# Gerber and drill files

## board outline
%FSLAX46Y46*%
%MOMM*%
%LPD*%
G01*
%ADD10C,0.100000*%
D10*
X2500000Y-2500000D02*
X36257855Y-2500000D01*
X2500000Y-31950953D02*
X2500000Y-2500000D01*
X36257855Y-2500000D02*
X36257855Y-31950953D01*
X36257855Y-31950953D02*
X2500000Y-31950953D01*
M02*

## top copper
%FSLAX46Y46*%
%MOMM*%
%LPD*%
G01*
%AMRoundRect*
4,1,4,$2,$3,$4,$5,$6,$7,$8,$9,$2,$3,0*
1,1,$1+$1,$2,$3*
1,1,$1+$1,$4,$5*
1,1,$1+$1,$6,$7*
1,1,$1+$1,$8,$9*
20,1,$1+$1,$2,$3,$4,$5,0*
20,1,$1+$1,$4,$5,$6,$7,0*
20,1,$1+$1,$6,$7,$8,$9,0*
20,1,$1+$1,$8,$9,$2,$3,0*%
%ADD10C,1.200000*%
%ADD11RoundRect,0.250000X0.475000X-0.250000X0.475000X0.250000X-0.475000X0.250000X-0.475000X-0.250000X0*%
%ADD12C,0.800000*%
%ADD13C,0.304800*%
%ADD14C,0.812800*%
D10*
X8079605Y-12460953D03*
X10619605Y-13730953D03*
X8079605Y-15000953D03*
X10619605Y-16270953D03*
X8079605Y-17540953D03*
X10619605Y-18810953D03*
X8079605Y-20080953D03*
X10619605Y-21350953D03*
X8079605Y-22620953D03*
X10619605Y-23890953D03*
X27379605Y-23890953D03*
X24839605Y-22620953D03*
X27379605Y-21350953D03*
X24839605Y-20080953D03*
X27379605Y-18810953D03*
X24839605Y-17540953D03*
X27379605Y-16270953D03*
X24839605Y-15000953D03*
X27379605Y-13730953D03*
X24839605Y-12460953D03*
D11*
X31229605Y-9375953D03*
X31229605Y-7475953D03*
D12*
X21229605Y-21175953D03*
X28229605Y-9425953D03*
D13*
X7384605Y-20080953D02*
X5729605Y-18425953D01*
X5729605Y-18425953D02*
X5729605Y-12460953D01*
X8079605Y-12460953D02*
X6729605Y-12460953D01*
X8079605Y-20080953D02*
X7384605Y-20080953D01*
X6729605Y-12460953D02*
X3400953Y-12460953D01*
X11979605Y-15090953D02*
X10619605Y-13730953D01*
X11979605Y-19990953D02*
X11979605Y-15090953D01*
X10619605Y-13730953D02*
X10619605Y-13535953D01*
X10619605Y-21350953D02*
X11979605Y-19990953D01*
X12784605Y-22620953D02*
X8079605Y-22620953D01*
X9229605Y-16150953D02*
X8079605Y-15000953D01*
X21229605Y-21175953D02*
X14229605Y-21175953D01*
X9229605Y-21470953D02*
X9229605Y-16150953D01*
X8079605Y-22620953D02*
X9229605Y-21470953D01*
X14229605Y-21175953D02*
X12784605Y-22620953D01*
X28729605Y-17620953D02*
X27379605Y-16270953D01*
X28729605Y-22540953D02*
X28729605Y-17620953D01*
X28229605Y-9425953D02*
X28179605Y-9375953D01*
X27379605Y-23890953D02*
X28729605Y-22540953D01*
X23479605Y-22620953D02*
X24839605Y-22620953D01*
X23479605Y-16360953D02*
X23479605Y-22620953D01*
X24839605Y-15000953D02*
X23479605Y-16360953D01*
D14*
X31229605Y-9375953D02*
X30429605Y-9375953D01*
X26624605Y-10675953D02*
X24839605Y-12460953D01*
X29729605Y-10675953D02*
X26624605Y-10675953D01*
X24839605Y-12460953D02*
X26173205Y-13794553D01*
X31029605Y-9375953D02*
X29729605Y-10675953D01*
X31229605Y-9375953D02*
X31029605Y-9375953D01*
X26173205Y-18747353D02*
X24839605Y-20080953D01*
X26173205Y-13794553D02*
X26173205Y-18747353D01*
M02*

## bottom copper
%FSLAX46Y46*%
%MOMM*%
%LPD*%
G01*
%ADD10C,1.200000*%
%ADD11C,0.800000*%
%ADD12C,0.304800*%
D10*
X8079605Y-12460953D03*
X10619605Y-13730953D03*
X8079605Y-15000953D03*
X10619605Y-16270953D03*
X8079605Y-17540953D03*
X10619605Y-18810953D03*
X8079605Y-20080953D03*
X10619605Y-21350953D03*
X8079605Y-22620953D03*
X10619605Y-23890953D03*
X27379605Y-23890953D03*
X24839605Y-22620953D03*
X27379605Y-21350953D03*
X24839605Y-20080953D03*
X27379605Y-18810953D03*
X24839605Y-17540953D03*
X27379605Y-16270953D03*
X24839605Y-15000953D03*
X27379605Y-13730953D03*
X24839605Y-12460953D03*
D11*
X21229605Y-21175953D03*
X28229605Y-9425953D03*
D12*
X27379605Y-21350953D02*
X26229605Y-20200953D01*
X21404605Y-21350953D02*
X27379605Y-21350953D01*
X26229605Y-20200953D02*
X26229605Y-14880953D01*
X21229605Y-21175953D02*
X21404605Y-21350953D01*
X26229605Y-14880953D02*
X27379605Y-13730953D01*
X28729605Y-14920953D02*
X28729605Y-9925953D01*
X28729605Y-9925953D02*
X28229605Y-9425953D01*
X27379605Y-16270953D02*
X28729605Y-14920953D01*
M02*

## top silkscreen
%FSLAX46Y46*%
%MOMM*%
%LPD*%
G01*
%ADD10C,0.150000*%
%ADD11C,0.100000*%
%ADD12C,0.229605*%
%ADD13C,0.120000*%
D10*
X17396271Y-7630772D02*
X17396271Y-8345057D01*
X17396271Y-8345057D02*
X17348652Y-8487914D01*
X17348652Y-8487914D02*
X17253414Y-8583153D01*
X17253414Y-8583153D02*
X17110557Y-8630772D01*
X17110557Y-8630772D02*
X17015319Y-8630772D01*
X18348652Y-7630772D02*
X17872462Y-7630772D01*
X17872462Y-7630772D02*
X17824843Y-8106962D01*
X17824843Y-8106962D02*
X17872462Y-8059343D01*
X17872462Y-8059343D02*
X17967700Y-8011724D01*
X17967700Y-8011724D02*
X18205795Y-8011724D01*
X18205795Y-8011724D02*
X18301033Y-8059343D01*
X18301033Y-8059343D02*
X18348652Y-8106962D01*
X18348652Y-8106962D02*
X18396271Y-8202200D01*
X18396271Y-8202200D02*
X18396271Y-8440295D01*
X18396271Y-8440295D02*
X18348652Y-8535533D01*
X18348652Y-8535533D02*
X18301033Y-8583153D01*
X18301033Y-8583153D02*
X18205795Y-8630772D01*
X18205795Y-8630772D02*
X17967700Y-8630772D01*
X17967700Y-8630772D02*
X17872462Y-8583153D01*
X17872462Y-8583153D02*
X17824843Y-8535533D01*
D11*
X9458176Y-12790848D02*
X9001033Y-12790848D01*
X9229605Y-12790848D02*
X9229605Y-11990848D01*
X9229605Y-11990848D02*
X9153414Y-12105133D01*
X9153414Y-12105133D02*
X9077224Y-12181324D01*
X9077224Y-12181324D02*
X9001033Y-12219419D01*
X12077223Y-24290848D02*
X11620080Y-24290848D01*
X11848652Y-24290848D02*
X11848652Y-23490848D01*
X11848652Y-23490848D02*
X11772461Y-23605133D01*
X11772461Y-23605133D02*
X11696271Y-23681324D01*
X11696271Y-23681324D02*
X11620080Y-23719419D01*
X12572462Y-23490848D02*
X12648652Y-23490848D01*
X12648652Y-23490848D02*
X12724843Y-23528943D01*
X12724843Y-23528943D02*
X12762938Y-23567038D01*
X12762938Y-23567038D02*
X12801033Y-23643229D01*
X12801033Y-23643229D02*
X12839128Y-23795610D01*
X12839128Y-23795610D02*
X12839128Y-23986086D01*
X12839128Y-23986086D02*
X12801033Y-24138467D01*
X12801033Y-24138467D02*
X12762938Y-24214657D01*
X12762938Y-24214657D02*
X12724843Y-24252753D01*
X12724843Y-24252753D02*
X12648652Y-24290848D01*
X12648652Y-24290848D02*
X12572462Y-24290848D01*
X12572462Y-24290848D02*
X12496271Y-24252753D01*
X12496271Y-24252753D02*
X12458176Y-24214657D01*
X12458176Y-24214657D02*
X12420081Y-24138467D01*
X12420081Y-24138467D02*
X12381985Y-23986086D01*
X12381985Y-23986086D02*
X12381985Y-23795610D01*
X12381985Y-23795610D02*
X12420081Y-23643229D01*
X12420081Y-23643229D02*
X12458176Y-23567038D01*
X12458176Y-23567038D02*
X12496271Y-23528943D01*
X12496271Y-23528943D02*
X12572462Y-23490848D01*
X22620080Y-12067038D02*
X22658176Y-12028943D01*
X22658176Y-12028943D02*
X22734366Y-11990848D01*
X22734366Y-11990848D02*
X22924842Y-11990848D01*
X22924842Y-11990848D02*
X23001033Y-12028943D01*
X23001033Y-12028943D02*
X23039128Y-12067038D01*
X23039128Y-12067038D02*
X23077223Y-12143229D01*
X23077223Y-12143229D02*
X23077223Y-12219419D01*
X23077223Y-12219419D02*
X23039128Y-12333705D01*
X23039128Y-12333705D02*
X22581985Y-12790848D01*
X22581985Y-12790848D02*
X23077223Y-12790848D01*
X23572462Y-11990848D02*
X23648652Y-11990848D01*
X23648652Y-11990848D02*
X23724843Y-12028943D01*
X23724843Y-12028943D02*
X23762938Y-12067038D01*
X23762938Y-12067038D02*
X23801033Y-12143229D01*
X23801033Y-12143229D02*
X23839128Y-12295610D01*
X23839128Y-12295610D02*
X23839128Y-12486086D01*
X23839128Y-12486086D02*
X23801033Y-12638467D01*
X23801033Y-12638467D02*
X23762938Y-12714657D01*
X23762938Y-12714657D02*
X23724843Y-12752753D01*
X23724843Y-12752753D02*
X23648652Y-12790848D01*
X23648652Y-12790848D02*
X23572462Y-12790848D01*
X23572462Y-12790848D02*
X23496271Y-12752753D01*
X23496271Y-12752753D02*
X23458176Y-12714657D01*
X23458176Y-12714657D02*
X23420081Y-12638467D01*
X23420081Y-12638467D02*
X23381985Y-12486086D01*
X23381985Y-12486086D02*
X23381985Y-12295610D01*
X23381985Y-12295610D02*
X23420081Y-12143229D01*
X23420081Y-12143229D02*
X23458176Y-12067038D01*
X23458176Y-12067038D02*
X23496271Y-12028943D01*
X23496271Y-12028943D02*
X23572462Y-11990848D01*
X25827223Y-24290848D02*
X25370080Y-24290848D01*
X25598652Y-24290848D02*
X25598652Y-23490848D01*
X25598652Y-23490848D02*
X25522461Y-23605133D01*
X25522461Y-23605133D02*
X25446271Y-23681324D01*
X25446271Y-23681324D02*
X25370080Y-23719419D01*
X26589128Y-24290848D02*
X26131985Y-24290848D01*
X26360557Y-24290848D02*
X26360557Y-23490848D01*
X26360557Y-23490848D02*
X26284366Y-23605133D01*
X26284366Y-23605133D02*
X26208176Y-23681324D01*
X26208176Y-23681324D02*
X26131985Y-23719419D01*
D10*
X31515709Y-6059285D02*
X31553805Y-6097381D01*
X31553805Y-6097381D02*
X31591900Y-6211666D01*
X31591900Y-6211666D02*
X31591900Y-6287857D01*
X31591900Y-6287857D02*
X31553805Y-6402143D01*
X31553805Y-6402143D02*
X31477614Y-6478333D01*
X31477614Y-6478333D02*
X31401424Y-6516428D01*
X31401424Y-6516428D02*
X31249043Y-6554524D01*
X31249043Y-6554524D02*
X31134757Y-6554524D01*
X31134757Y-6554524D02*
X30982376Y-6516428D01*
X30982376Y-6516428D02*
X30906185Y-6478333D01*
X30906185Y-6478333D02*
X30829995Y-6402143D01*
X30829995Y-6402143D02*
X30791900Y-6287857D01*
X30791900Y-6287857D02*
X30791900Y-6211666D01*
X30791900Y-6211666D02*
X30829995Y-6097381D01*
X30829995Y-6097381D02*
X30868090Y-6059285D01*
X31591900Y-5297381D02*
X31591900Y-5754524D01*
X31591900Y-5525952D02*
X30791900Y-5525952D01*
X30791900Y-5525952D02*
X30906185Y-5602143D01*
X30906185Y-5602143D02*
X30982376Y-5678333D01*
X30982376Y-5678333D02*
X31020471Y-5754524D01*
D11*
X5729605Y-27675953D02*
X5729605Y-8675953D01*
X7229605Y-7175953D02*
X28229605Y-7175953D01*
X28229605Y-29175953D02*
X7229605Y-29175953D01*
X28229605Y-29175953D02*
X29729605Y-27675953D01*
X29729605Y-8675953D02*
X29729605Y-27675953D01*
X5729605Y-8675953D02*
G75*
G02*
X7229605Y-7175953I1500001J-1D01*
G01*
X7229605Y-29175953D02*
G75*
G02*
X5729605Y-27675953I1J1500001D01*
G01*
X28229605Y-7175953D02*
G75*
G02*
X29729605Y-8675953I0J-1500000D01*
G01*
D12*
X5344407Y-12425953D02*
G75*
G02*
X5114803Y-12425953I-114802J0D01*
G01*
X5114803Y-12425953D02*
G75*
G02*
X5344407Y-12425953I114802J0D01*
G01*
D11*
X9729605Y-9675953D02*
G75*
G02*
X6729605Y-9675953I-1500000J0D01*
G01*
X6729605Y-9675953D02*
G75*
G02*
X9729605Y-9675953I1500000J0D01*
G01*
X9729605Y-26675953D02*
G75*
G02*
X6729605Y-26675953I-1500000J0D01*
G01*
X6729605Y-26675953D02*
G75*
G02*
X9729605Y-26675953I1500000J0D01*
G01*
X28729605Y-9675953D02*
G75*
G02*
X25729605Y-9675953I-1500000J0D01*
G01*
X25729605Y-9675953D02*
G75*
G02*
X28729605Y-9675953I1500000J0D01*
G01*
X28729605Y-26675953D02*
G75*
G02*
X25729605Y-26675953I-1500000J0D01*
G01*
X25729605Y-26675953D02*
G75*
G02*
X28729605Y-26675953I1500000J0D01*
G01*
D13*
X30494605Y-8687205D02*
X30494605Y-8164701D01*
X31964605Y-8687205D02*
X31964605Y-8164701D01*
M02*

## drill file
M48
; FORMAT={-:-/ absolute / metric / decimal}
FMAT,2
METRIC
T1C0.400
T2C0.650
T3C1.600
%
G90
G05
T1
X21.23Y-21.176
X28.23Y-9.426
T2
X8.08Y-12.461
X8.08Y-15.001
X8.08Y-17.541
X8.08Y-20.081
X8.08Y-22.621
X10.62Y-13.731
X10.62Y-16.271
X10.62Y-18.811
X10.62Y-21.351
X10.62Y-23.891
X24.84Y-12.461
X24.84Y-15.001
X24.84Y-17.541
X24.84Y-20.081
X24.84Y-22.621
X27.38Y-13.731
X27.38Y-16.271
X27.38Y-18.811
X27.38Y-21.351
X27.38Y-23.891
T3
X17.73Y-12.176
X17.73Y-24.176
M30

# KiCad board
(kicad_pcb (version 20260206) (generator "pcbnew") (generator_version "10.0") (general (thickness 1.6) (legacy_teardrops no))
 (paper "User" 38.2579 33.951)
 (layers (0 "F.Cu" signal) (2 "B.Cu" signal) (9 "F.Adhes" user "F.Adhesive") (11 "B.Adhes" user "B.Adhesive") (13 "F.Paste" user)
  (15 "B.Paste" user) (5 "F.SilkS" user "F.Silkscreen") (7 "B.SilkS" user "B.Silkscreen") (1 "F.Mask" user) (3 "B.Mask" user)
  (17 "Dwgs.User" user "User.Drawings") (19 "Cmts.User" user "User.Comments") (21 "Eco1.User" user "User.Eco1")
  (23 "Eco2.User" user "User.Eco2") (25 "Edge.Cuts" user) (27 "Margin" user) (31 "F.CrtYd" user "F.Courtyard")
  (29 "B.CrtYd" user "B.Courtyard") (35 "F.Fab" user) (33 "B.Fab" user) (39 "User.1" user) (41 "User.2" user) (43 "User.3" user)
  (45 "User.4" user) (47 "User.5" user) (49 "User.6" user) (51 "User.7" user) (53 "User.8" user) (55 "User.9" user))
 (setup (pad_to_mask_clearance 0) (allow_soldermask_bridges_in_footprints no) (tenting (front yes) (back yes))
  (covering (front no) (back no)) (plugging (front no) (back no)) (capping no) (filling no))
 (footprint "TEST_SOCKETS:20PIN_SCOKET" (layer "F.Cu") (at 17.729605 18.175953)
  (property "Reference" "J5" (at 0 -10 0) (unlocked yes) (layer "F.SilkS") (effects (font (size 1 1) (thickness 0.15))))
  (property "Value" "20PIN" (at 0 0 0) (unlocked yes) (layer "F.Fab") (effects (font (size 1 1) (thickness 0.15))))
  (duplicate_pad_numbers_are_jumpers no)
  (fp_line (start -12 9.5) (end -12 -9.5) (stroke (width 0.1) (type default)) (layer "F.SilkS"))
  (fp_line (start -10.5 -11) (end 10.5 -11) (stroke (width 0.1) (type default)) (layer "F.SilkS"))
  (fp_line (start 10.5 11) (end -10.5 11) (stroke (width 0.1) (type default)) (layer "F.SilkS"))
  (fp_line (start 10.5 11) (end 12 9.5) (stroke (width 0.1) (type default)) (layer "F.SilkS"))
  (fp_line (start 12 -9.5) (end 12 9.5) (stroke (width 0.1) (type default)) (layer "F.SilkS"))
  (fp_arc (start -12 -9.5) (mid -11.56066 -10.56066) (end -10.5 -11) (stroke (width 0.1) (type default)) (layer "F.SilkS"))
  (fp_arc (start -10.5 11) (mid -11.56066 10.56066) (end -12 9.5) (stroke (width 0.1) (type default)) (layer "F.SilkS"))
  (fp_arc (start 10.5 -11) (mid 11.56066 -10.56066) (end 12 -9.5) (stroke (width 0.1) (type default)) (layer "F.SilkS"))
  (fp_circle (center -12.5 -5.75) (end -12.320395 -5.75) (stroke (width 0.1) (type solid)) (fill yes) (layer "F.SilkS"))
  (fp_circle (center -9.5 -8.5) (end -8 -8.5) (stroke (width 0.1) (type default)) (fill no) (layer "F.SilkS"))
  (fp_circle (center -9.5 8.5) (end -8 8.5) (stroke (width 0.1) (type default)) (fill no) (layer "F.SilkS"))
  (fp_circle (center 9.5 -8.5) (end 8 -8.5) (stroke (width 0.1) (type default)) (fill no) (layer "F.SilkS"))
  (fp_circle (center 9.5 8.5) (end 8 8.5) (stroke (width 0.1) (type default)) (fill no) (layer "F.SilkS"))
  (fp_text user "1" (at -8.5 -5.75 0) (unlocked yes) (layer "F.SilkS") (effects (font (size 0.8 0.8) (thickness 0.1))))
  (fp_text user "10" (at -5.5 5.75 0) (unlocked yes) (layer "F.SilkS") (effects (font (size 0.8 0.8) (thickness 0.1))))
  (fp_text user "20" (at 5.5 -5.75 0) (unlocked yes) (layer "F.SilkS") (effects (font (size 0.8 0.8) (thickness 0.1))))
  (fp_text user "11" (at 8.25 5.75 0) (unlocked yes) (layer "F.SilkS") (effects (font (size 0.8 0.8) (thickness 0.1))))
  (pad "" np_thru_hole circle (at 0 -6) (size 1.6 1.6) (drill 1.6) (layers "*.Cu" "*.Mask"))
  (pad "" np_thru_hole circle (at 0 6) (size 1.6 1.6) (drill 1.6) (layers "*.Cu" "*.Mask"))
  (pad "1" thru_hole circle (at -9.65 -5.715) (size 1.2 1.2) (drill 0.65) (layers "*.Cu" "*.Mask") (remove_unused_layers no) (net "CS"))
  (pad "2" thru_hole circle (at -7.11 -4.445) (size 1.2 1.2) (drill 0.65) (layers "*.Cu" "*.Mask") (remove_unused_layers no) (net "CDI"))
  (pad "3" thru_hole circle (at -9.65 -3.175) (size 1.2 1.2) (drill 0.65) (layers "*.Cu" "*.Mask") (remove_unused_layers no) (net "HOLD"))
  (pad "4" thru_hole circle (at -7.11 -1.905) (size 1.2 1.2) (drill 0.65) (layers "*.Cu" "*.Mask") (remove_unused_layers no)
   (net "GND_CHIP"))
  (pad "5" thru_hole circle (at -9.65 -0.635) (size 1.2 1.2) (drill 0.65) (layers "*.Cu" "*.Mask") (remove_unused_layers no)
   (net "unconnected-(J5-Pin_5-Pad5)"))
  (pad "6" thru_hole circle (at -7.11 0.635) (size 1.2 1.2) (drill 0.65) (layers "*.Cu" "*.Mask") (remove_unused_layers no)
   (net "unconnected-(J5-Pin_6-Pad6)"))
  (pad "7" thru_hole circle (at -9.65 1.905) (size 1.2 1.2) (drill 0.65) (layers "*.Cu" "*.Mask") (remove_unused_layers no) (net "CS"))
  (pad "8" thru_hole circle (at -7.11 3.175) (size 1.2 1.2) (drill 0.65) (layers "*.Cu" "*.Mask") (remove_unused_layers no) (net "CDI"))
  (pad "9" thru_hole circle (at -9.65 4.445) (size 1.2 1.2) (drill 0.65) (layers "*.Cu" "*.Mask") (remove_unused_layers no) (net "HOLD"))
  (pad "10" thru_hole circle (at -7.11 5.715) (size 1.2 1.2) (drill 0.65) (layers "*.Cu" "*.Mask") (remove_unused_layers no)
   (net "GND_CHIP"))
  (pad "11" thru_hole circle (at 9.65 5.715 180) (size 1.2 1.2) (drill 0.65) (layers "*.Cu" "*.Mask") (remove_unused_layers no) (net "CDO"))
  (pad "12" thru_hole circle (at 7.11 4.445 180) (size 1.2 1.2) (drill 0.65) (layers "*.Cu" "*.Mask") (remove_unused_layers no) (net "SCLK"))
  (pad "13" thru_hole circle (at 9.65 3.175 180) (size 1.2 1.2) (drill 0.65) (layers "*.Cu" "*.Mask") (remove_unused_layers no) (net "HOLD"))
  (pad "14" thru_hole circle (at 7.11 1.905 180) (size 1.2 1.2) (drill 0.65) (layers "*.Cu" "*.Mask") (remove_unused_layers no)
   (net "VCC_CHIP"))
  (pad "15" thru_hole circle (at 9.65 0.635 180) (size 1.2 1.2) (drill 0.65) (layers "*.Cu" "*.Mask") (remove_unused_layers no)
   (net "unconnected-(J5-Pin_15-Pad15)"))
  (pad "16" thru_hole circle (at 7.11 -0.635 180) (size 1.2 1.2) (drill 0.65) (layers "*.Cu" "*.Mask") (remove_unused_layers no)
   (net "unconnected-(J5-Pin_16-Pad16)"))
  (pad "17" thru_hole circle (at 9.65 -1.905 180) (size 1.2 1.2) (drill 0.65) (layers "*.Cu" "*.Mask") (remove_unused_layers no) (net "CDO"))
  (pad "18" thru_hole circle (at 7.11 -3.175 180) (size 1.2 1.2) (drill 0.65) (layers "*.Cu" "*.Mask") (remove_unused_layers no)
   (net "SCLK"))
  (pad "19" thru_hole circle (at 9.65 -4.445 180) (size 1.2 1.2) (drill 0.65) (layers "*.Cu" "*.Mask") (remove_unused_layers no)
   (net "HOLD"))
  (pad "20" thru_hole circle (at 7.11 -5.715 180) (size 1.2 1.2) (drill 0.65) (layers "*.Cu" "*.Mask") (remove_unused_layers no)
   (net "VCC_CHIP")))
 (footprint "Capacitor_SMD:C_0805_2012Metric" (layer "F.Cu") (at 31.229605 8.425953 90)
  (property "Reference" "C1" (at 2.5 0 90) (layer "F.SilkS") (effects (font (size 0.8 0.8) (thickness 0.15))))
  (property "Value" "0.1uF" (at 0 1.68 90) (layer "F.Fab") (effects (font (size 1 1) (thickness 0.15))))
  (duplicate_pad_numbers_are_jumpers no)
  (fp_line (start -0.261252 -0.735) (end 0.261252 -0.735) (stroke (width 0.12) (type solid)) (layer "F.SilkS"))
  (fp_line (start -0.261252 0.735) (end 0.261252 0.735) (stroke (width 0.12) (type solid)) (layer "F.SilkS"))
  (pad "1" smd roundrect (at -0.95 0 90) (size 1 1.45) (layers "F.Cu" "F.Mask" "F.Paste") (roundrect_rratio 0.25) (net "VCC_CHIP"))
  (pad "2" smd roundrect (at 0.95 0 90) (size 1 1.45) (layers "F.Cu" "F.Mask" "F.Paste") (roundrect_rratio 0.25) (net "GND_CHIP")))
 (gr_line (start 2.5 2.5) (end 36.257855 2.5) (stroke (width 0.1) (type default)) (layer "Edge.Cuts"))
 (gr_line (start 2.5 31.950953) (end 2.5 2.5) (stroke (width 0.1) (type default)) (layer "Edge.Cuts"))
 (gr_line (start 36.257855 2.5) (end 36.257855 31.950953) (stroke (width 0.1) (type default)) (layer "Edge.Cuts"))
 (gr_line (start 36.257855 31.950953) (end 2.5 31.950953) (stroke (width 0.1) (type default)) (layer "Edge.Cuts"))
 (segment (start 7.384605 20.080953) (end 5.729605 18.425953) (width 0.3048) (layer "F.Cu") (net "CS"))
 (segment (start 5.729605 18.425953) (end 5.729605 12.460953) (width 0.3048) (layer "F.Cu") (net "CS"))
 (segment (start 8.079605 12.460953) (end 6.729605 12.460953) (width 0.3048) (layer "F.Cu") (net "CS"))
 (segment (start 8.079605 20.080953) (end 7.384605 20.080953) (width 0.3048) (layer "F.Cu") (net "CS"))
 (segment (start 6.729605 12.460953) (end 3.400953 12.460953) (width 0.3048) (layer "F.Cu") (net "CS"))
 (segment (start 11.979605 15.090953) (end 10.619605 13.730953) (width 0.3048) (layer "F.Cu") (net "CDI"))
 (segment (start 11.979605 19.990953) (end 11.979605 15.090953) (width 0.3048) (layer "F.Cu") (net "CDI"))
 (segment (start 10.619605 13.730953) (end 10.619605 13.535953) (width 0.3048) (layer "F.Cu") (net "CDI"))
 (segment (start 10.619605 21.350953) (end 11.979605 19.990953) (width 0.3048) (layer "F.Cu") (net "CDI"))
 (segment (start 12.784605 22.620953) (end 8.079605 22.620953) (width 0.3048) (layer "F.Cu") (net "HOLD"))
 (segment (start 9.229605 16.150953) (end 8.079605 15.000953) (width 0.3048) (layer "F.Cu") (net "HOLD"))
 (segment (start 21.229605 21.175953) (end 14.229605 21.175953) (width 0.3048) (layer "F.Cu") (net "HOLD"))
 (segment (start 9.229605 21.470953) (end 9.229605 16.150953) (width 0.3048) (layer "F.Cu") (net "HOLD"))
 (segment (start 8.079605 22.620953) (end 9.229605 21.470953) (width 0.3048) (layer "F.Cu") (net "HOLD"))
 (segment (start 14.229605 21.175953) (end 12.784605 22.620953) (width 0.3048) (layer "F.Cu") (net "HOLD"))
 (via (at 21.229605 21.175953) (size 0.8) (drill 0.4) (layers "F.Cu" "B.Cu") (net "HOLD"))
 (segment (start 27.379605 21.350953) (end 26.229605 20.200953) (width 0.3048) (layer "B.Cu") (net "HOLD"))
 (segment (start 21.404605 21.350953) (end 27.379605 21.350953) (width 0.3048) (layer "B.Cu") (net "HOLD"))
 (segment (start 26.229605 20.200953) (end 26.229605 14.880953) (width 0.3048) (layer "B.Cu") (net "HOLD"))
 (segment (start 21.229605 21.175953) (end 21.404605 21.350953) (width 0.3048) (layer "B.Cu") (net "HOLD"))
 (segment (start 26.229605 14.880953) (end 27.379605 13.730953) (width 0.3048) (layer "B.Cu") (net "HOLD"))
 (segment (start 28.729605 17.620953) (end 27.379605 16.270953) (width 0.3048) (layer "F.Cu") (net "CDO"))
 (segment (start 28.729605 22.540953) (end 28.729605 17.620953) (width 0.3048) (layer "F.Cu") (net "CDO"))
 (segment (start 28.229605 9.425953) (end 28.179605 9.375953) (width 0.3048) (layer "F.Cu") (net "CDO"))
 (segment (start 27.379605 23.890953) (end 28.729605 22.540953) (width 0.3048) (layer "F.Cu") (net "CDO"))
 (via (at 28.229605 9.425953) (size 0.8) (drill 0.4) (layers "F.Cu" "B.Cu") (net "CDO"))
 (segment (start 28.729605 14.920953) (end 28.729605 9.925953) (width 0.3048) (layer "B.Cu") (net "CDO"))
 (segment (start 28.729605 9.925953) (end 28.229605 9.425953) (width 0.3048) (layer "B.Cu") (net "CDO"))
 (segment (start 27.379605 16.270953) (end 28.729605 14.920953) (width 0.3048) (layer "B.Cu") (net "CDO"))
 (segment (start 23.479605 22.620953) (end 24.839605 22.620953) (width 0.3048) (layer "F.Cu") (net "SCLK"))
 (segment (start 23.479605 16.360953) (end 23.479605 22.620953) (width 0.3048) (layer "F.Cu") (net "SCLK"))
 (segment (start 24.839605 15.000953) (end 23.479605 16.360953) (width 0.3048) (layer "F.Cu") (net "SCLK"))
 (segment (start 31.229605 9.375953) (end 30.429605 9.375953) (width 0.8128) (layer "F.Cu") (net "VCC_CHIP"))
 (segment (start 26.624605 10.675953) (end 24.839605 12.460953) (width 0.8128) (layer "F.Cu") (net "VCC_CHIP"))
 (segment (start 29.729605 10.675953) (end 26.624605 10.675953) (width 0.8128) (layer "F.Cu") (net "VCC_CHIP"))
 (segment (start 24.839605 12.460953) (end 26.173205 13.794553) (width 0.8128) (layer "F.Cu") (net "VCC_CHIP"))
 (segment (start 31.029605 9.375953) (end 29.729605 10.675953) (width 0.8128) (layer "F.Cu") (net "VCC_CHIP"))
 (segment (start 31.229605 9.375953) (end 31.029605 9.375953) (width 0.8128) (layer "F.Cu") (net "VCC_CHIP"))
 (segment (start 26.173205 18.747353) (end 24.839605 20.080953) (width 0.8128) (layer "F.Cu") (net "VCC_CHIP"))
 (segment (start 26.173205 13.794553) (end 26.173205 18.747353) (width 0.8128) (layer "F.Cu") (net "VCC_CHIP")))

